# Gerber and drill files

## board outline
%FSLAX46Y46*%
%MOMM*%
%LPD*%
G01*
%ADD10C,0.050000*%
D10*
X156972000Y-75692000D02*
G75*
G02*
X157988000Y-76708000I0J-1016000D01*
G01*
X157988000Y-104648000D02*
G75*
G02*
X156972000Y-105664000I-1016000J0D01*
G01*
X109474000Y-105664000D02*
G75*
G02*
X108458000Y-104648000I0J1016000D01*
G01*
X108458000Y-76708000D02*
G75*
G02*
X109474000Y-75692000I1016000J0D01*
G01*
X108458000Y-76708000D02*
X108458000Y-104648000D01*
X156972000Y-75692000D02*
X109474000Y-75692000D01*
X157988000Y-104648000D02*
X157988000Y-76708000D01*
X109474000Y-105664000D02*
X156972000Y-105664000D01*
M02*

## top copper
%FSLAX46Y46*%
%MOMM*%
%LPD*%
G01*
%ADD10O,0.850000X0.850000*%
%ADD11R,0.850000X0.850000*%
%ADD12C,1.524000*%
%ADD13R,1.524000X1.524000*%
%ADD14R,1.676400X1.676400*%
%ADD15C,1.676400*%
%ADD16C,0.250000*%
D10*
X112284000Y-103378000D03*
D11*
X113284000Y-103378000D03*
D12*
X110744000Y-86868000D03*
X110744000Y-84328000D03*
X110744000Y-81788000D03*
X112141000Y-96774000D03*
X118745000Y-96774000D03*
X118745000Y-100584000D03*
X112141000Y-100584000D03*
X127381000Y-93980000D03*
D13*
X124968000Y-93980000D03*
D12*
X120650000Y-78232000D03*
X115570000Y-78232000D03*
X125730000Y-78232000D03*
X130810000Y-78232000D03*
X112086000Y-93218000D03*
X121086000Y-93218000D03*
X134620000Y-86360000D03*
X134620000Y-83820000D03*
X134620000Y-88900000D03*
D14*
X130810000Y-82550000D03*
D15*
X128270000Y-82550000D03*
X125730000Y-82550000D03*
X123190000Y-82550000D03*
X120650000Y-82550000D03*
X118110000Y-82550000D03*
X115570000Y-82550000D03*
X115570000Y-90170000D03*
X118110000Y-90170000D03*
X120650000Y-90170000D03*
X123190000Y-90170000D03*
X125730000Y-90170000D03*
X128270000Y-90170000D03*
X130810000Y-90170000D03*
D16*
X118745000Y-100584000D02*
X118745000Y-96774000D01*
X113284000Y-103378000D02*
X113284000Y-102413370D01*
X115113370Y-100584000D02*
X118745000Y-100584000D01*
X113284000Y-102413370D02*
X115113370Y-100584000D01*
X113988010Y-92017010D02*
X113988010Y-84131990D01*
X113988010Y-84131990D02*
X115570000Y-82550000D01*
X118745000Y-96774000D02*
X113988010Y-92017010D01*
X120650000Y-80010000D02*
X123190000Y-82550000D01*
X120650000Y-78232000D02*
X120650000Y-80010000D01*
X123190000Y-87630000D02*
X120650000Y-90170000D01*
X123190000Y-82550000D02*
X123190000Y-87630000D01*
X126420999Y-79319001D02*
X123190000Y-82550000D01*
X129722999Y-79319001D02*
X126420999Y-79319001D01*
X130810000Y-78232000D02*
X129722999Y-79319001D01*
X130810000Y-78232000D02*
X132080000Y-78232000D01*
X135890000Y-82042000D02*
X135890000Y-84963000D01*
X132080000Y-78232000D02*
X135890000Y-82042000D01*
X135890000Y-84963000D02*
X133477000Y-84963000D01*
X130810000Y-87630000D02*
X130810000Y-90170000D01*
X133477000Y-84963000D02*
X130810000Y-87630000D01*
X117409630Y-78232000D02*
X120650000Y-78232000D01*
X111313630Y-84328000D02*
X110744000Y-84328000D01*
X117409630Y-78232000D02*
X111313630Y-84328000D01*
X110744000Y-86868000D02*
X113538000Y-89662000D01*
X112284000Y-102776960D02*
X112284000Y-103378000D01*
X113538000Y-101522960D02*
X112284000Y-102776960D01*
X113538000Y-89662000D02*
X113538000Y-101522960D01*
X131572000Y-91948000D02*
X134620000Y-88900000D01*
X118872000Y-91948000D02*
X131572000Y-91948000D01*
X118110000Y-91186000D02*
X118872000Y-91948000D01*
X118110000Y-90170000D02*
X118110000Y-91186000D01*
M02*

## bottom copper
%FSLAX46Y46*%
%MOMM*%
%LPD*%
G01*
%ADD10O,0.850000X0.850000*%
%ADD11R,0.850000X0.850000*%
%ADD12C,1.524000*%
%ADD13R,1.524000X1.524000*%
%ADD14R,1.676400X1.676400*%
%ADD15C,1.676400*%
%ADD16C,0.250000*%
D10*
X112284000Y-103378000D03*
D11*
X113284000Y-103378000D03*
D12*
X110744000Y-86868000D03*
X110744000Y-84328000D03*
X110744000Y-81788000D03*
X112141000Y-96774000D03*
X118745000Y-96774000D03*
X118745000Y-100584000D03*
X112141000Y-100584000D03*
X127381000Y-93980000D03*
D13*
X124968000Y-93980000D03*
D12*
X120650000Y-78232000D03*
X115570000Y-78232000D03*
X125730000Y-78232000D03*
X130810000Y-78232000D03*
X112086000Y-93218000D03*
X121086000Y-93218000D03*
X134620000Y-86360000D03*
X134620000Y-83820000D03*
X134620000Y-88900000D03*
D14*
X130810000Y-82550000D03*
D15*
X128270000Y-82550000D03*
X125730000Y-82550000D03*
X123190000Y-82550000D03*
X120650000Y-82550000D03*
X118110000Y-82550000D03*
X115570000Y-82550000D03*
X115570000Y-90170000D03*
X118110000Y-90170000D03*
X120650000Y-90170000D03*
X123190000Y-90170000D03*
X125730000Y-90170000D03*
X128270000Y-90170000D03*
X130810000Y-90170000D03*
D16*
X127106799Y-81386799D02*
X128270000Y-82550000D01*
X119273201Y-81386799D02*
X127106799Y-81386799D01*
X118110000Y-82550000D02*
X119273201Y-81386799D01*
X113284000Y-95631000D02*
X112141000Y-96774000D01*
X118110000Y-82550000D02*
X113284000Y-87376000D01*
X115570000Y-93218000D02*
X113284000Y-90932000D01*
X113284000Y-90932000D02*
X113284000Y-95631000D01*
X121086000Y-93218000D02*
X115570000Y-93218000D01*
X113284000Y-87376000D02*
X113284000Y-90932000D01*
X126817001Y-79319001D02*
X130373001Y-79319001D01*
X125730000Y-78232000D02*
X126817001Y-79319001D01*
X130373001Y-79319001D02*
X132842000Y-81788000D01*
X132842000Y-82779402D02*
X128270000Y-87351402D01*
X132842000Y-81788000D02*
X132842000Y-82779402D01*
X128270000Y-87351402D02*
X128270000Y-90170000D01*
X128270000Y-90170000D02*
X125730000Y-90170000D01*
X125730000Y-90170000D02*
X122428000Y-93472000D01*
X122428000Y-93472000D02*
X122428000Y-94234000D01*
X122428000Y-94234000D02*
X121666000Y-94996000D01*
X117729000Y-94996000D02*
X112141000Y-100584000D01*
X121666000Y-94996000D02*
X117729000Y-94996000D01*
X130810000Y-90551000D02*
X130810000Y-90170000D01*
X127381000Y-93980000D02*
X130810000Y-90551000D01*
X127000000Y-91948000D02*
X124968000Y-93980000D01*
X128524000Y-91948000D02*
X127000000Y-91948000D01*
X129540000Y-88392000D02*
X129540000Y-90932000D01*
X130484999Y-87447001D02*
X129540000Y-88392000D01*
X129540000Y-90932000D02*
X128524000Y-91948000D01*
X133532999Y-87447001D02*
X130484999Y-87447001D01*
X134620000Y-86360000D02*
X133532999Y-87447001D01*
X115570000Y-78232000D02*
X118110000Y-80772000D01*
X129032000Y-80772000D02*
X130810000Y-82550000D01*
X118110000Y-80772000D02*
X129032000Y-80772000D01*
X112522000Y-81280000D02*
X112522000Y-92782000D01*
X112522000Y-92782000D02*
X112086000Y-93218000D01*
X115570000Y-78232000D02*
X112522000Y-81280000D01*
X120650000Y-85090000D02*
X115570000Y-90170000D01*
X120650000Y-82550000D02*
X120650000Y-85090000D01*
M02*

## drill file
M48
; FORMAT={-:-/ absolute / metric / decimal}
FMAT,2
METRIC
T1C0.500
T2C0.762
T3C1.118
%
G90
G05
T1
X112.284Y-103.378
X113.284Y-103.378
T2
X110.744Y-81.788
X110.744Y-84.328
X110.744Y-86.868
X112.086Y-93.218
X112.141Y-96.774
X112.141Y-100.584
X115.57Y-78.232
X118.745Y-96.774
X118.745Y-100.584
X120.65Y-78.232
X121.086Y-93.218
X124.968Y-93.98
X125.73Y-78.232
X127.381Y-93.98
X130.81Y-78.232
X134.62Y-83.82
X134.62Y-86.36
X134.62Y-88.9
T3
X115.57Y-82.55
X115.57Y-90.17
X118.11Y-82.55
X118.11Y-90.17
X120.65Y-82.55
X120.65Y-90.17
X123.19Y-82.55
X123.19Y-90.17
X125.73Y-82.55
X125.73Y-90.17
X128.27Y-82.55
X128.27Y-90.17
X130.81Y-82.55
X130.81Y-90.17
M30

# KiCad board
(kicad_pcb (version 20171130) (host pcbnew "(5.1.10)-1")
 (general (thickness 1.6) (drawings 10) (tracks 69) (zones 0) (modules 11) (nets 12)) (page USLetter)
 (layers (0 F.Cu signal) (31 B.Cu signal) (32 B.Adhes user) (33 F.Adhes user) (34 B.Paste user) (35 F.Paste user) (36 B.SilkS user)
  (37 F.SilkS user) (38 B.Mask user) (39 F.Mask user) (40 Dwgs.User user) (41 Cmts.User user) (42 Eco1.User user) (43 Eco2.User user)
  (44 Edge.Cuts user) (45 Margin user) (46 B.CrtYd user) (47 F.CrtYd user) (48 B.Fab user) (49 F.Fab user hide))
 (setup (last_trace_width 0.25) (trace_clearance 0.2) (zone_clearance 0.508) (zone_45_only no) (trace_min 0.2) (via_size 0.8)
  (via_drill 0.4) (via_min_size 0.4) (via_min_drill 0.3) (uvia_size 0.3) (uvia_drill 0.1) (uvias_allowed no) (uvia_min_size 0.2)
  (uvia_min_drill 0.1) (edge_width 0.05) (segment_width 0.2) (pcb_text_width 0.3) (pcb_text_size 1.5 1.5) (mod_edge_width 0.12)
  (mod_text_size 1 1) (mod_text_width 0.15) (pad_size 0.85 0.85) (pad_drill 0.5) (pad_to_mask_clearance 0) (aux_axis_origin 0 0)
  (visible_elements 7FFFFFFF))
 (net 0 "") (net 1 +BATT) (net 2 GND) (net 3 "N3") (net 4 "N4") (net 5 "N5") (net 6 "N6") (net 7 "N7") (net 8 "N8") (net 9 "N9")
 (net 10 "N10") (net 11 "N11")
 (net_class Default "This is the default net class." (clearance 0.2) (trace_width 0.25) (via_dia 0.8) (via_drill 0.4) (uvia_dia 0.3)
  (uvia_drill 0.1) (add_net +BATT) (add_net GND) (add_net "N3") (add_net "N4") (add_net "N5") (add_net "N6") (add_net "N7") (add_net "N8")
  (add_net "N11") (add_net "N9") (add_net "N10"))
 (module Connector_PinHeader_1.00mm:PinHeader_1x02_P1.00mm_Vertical (layer F.Cu) (at 113.284 103.378 270)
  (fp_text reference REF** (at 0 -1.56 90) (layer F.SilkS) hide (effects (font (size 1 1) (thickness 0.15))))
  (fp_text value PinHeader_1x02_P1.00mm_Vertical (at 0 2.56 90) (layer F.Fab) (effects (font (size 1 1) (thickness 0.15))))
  (pad 2 thru_hole oval (at 0 1 270) (size 0.85 0.85) (drill 0.5) (layers *.Cu *.Mask) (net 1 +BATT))
  (pad 1 thru_hole rect (at 0 0 270) (size 0.85 0.85) (drill 0.5) (layers *.Cu *.Mask) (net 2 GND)))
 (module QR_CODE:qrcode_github (layer F.Cu) (at 146.304 89.916)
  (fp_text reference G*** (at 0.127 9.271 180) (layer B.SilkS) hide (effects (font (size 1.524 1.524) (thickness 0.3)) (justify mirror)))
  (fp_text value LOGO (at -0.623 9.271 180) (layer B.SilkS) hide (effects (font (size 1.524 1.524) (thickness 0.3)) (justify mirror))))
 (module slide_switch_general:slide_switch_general (layer F.Cu) (at 110.744 84.328 270)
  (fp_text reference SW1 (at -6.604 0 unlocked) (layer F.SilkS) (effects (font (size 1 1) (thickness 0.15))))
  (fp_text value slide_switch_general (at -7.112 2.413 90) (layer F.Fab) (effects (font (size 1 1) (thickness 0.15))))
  (pad 3 thru_hole circle (at 2.54 0 270) (size 1.524 1.524) (drill 0.762) (layers *.Cu *.Mask) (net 1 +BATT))
  (pad 2 thru_hole circle (at 0 0 270) (size 1.524 1.524) (drill 0.762) (layers *.Cu *.Mask) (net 1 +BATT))
  (pad 1 thru_hole circle (at -2.54 0 270) (size 1.524 1.524) (drill 0.762) (layers *.Cu *.Mask)))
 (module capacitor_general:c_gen (layer F.Cu) (at 115.57 96.774)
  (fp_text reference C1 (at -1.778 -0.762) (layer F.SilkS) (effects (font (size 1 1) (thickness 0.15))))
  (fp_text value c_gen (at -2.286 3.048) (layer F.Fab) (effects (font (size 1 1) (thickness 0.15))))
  (pad 1 thru_hole circle (at -3.429 0) (size 1.524 1.524) (drill 0.762) (layers *.Cu *.Mask) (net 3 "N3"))
  (pad 2 thru_hole circle (at 3.175 0) (size 1.524 1.524) (drill 0.762) (layers *.Cu *.Mask) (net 2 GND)))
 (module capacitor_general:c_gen (layer F.Cu) (at 115.57 100.584)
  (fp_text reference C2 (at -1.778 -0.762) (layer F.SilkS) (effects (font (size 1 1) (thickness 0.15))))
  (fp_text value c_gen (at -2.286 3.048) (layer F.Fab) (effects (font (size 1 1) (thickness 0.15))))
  (pad 2 thru_hole circle (at 3.175 0) (size 1.524 1.524) (drill 0.762) (layers *.Cu *.Mask) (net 2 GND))
  (pad 1 thru_hole circle (at -3.429 0) (size 1.524 1.524) (drill 0.762) (layers *.Cu *.Mask) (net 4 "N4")))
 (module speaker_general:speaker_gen (layer F.Cu) (at 126.238 93.98 180)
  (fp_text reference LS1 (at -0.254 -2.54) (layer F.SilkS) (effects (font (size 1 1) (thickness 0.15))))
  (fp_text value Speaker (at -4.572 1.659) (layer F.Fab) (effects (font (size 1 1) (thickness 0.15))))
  (pad 1 thru_hole circle (at -1.143 0 180) (size 1.524 1.524) (drill 0.762) (layers *.Cu *.Mask) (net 1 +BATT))
  (pad 2 thru_hole rect (at 1.27 0 180) (size 1.524 1.524) (drill 0.762) (layers *.Cu *.Mask) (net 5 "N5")))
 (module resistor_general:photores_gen (layer F.Cu) (at 118.11 78.232 180)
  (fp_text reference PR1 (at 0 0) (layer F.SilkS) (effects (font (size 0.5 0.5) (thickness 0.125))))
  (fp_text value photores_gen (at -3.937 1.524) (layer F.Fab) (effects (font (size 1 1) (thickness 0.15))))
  (pad 1 thru_hole circle (at -2.54 0 180) (size 1.524 1.524) (drill 0.762) (layers *.Cu *.Mask) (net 1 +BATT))
  (pad 2 thru_hole circle (at 2.54 0 180) (size 1.524 1.524) (drill 0.762) (layers *.Cu *.Mask) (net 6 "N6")))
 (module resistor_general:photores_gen (layer F.Cu) (at 128.27 78.232 180)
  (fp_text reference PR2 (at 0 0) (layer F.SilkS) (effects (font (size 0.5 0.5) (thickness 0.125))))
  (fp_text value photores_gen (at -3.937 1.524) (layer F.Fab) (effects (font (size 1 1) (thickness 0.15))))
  (pad 2 thru_hole circle (at 2.54 0 180) (size 1.524 1.524) (drill 0.762) (layers *.Cu *.Mask) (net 4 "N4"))
  (pad 1 thru_hole circle (at -2.54 0 180) (size 1.524 1.524) (drill 0.762) (layers *.Cu *.Mask) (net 1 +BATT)))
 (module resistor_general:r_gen (layer F.Cu) (at 116.586 93.218)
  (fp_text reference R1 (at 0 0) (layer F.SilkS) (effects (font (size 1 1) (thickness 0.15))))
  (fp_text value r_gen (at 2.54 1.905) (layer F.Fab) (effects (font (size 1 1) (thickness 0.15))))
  (pad 1 thru_hole circle (at -4.5 0) (size 1.524 1.524) (drill 0.762) (layers *.Cu *.Mask) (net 6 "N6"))
  (pad 2 thru_hole circle (at 4.5 0) (size 1.524 1.524) (drill 0.762) (layers *.Cu *.Mask) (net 3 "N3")))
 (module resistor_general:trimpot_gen (layer F.Cu) (at 133.604 86.36 270)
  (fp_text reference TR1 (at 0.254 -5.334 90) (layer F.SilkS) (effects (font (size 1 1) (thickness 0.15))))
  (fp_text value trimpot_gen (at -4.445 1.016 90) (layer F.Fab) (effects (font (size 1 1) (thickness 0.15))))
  (pad 2 thru_hole circle (at 0 -1.016 270) (size 1.524 1.524) (drill 0.762) (layers *.Cu *.Mask) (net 5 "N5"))
  (pad 1 thru_hole circle (at -2.54 -1.016 270) (size 1.524 1.524) (drill 0.762) (layers *.Cu *.Mask) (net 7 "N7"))
  (pad 3 thru_hole circle (at 2.54 -1.016 270) (size 1.524 1.524) (drill 0.762) (layers *.Cu *.Mask) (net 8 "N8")))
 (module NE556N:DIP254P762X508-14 (layer F.Cu) (at 115.57 90.17 270)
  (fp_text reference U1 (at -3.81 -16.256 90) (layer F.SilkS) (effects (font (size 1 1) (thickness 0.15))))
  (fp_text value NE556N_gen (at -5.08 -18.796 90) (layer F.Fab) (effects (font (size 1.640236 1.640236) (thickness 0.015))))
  (pad 1 thru_hole rect (at -7.62 -15.24 270) (size 1.6764 1.6764) (drill 1.1176) (layers *.Cu *.Mask) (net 6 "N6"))
  (pad 2 thru_hole circle (at -7.62 -12.7 270) (size 1.6764 1.6764) (drill 1.1176) (layers *.Cu *.Mask) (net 3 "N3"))
  (pad 3 thru_hole circle (at -7.62 -10.16 270) (size 1.6764 1.6764) (drill 1.1176) (layers *.Cu *.Mask) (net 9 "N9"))
  (pad 4 thru_hole circle (at -7.62 -7.62 270) (size 1.6764 1.6764) (drill 1.1176) (layers *.Cu *.Mask) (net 1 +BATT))
  (pad 5 thru_hole circle (at -7.62 -5.08 270) (size 1.6764 1.6764) (drill 1.1176) (layers *.Cu *.Mask) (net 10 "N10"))
  (pad 6 thru_hole circle (at -7.62 -2.54 270) (size 1.6764 1.6764) (drill 1.1176) (layers *.Cu *.Mask) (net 3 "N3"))
  (pad 7 thru_hole circle (at -7.62 0 270) (size 1.6764 1.6764) (drill 1.1176) (layers *.Cu *.Mask) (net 2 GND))
  (pad 8 thru_hole circle (at 0 0 270) (size 1.6764 1.6764) (drill 1.1176) (layers *.Cu *.Mask) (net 10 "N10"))
  (pad 9 thru_hole circle (at 0 -2.54 270) (size 1.6764 1.6764) (drill 1.1176) (layers *.Cu *.Mask) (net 8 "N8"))
  (pad 10 thru_hole circle (at 0 -5.08 270) (size 1.6764 1.6764) (drill 1.1176) (layers *.Cu *.Mask) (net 1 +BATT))
  (pad 11 thru_hole circle (at 0 -7.62 270) (size 1.6764 1.6764) (drill 1.1176) (layers *.Cu *.Mask) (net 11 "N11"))
  (pad 12 thru_hole circle (at 0 -10.16 270) (size 1.6764 1.6764) (drill 1.1176) (layers *.Cu *.Mask) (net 4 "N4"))
  (pad 13 thru_hole circle (at 0 -12.7 270) (size 1.6764 1.6764) (drill 1.1176) (layers *.Cu *.Mask) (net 4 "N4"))
  (pad 14 thru_hole circle (at 0 -15.24 270) (size 1.6764 1.6764) (drill 1.1176) (layers *.Cu *.Mask) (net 1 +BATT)))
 (gr_arc (start 156.972 76.708) (end 157.988 76.708) (angle -90) (layer Edge.Cuts) (width 0.05))
 (gr_arc (start 156.972 104.648) (end 156.972 105.664) (angle -90) (layer Edge.Cuts) (width 0.05))
 (gr_arc (start 109.474 104.648) (end 108.458 104.648) (angle -90) (layer Edge.Cuts) (width 0.05))
 (gr_arc (start 109.474 76.708) (end 109.474 75.692) (angle -90) (layer Edge.Cuts) (width 0.05))
 (gr_line (start 108.458 76.708) (end 108.458 104.648) (layer Edge.Cuts) (width 0.05))
 (gr_line (start 156.972 75.692) (end 109.474 75.692) (layer Edge.Cuts) (width 0.05))
 (gr_line (start 157.988 104.648) (end 157.988 76.708) (layer Edge.Cuts) (width 0.05))
 (gr_line (start 109.474 105.664) (end 156.972 105.664) (layer Edge.Cuts) (width 0.05))
 (segment (start 127.106799 81.386799) (end 128.27 82.55) (width 0.25) (layer B.Cu) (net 3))
 (segment (start 119.273201 81.386799) (end 127.106799 81.386799) (width 0.25) (layer B.Cu) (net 3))
 (segment (start 118.11 82.55) (end 119.273201 81.386799) (width 0.25) (layer B.Cu) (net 3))
 (segment (start 113.284 95.631) (end 112.141 96.774) (width 0.25) (layer B.Cu) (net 3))
 (segment (start 118.11 82.55) (end 113.284 87.376) (width 0.25) (layer B.Cu) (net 3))
 (segment (start 115.57 93.218) (end 113.284 90.932) (width 0.25) (layer B.Cu) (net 3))
 (segment (start 113.284 90.932) (end 113.284 95.631) (width 0.25) (layer B.Cu) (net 3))
 (segment (start 121.086 93.218) (end 115.57 93.218) (width 0.25) (layer B.Cu) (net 3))
 (segment (start 113.284 87.376) (end 113.284 90.932) (width 0.25) (layer B.Cu) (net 3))
 (segment (start 118.745 100.584) (end 118.745 96.774) (width 0.25) (layer F.Cu) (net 2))
 (segment (start 113.284 103.378) (end 113.284 102.41337) (width 0.25) (layer F.Cu) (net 2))
 (segment (start 115.11337 100.584) (end 118.745 100.584) (width 0.25) (layer F.Cu) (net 2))
 (segment (start 113.284 102.41337) (end 115.11337 100.584) (width 0.25) (layer F.Cu) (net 2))
 (segment (start 113.98801 92.01701) (end 113.98801 84.13199) (width 0.25) (layer F.Cu) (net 2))
 (segment (start 113.98801 84.13199) (end 115.57 82.55) (width 0.25) (layer F.Cu) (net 2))
 (segment (start 118.745 96.774) (end 113.98801 92.01701) (width 0.25) (layer F.Cu) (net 2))
 (segment (start 126.817001 79.319001) (end 130.373001 79.319001) (width 0.25) (layer B.Cu) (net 4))
 (segment (start 125.73 78.232) (end 126.817001 79.319001) (width 0.25) (layer B.Cu) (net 4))
 (segment (start 130.373001 79.319001) (end 132.842 81.788) (width 0.25) (layer B.Cu) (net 4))
 (segment (start 132.842 82.779402) (end 128.27 87.351402) (width 0.25) (layer B.Cu) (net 4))
 (segment (start 132.842 81.788) (end 132.842 82.779402) (width 0.25) (layer B.Cu) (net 4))
 (segment (start 128.27 87.351402) (end 128.27 90.17) (width 0.25) (layer B.Cu) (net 4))
 (segment (start 128.27 90.17) (end 125.73 90.17) (width 0.25) (layer B.Cu) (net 4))
 (segment (start 125.73 90.17) (end 122.428 93.472) (width 0.25) (layer B.Cu) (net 4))
 (segment (start 122.428 93.472) (end 122.428 94.234) (width 0.25) (layer B.Cu) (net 4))
 (segment (start 122.428 94.234) (end 121.666 94.996) (width 0.25) (layer B.Cu) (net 4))
 (segment (start 117.729 94.996) (end 112.141 100.584) (width 0.25) (layer B.Cu) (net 4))
 (segment (start 121.666 94.996) (end 117.729 94.996) (width 0.25) (layer B.Cu) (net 4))
 (segment (start 120.65 80.01) (end 123.19 82.55) (width 0.25) (layer F.Cu) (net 1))
 (segment (start 120.65 78.232) (end 120.65 80.01) (width 0.25) (layer F.Cu) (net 1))
 (segment (start 123.19 87.63) (end 120.65 90.17) (width 0.25) (layer F.Cu) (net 1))
 (segment (start 123.19 82.55) (end 123.19 87.63) (width 0.25) (layer F.Cu) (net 1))
 (segment (start 126.420999 79.319001) (end 123.19 82.55) (width 0.25) (layer F.Cu) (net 1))
 (segment (start 129.722999 79.319001) (end 126.420999 79.319001) (width 0.25) (layer F.Cu) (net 1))
 (segment (start 130.81 78.232) (end 129.722999 79.319001) (width 0.25) (layer F.Cu) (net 1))
 (segment (start 130.81 78.232) (end 132.08 78.232) (width 0.25) (layer F.Cu) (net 1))
 (segment (start 135.89 82.042) (end 135.89 84.963) (width 0.25) (layer F.Cu) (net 1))
 (segment (start 132.08 78.232) (end 135.89 82.042) (width 0.25) (layer F.Cu) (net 1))
 (segment (start 135.89 84.963) (end 133.477 84.963) (width 0.25) (layer F.Cu) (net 1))
 (segment (start 130.81 87.63) (end 130.81 90.17) (width 0.25) (layer F.Cu) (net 1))
 (segment (start 133.477 84.963) (end 130.81 87.63) (width 0.25) (layer F.Cu) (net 1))
 (segment (start 130.81 90.551) (end 130.81 90.17) (width 0.25) (layer B.Cu) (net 1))
 (segment (start 127.381 93.98) (end 130.81 90.551) (width 0.25) (layer B.Cu) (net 1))
 (segment (start 117.40963 78.232) (end 120.65 78.232) (width 0.25) (layer F.Cu) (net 1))
 (segment (start 111.31363 84.328) (end 110.744 84.328) (width 0.25) (layer F.Cu) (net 1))
 (segment (start 117.40963 78.232) (end 111.31363 84.328) (width 0.25) (layer F.Cu) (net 1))
 (segment (start 110.744 86.868) (end 113.538 89.662) (width 0.25) (layer F.Cu) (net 1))
 (segment (start 112.284 102.77696) (end 112.284 103.378) (width 0.25) (layer F.Cu) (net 1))
 (segment (start 113.538 101.52296) (end 112.284 102.77696) (width 0.25) (layer F.Cu) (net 1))
 (segment (start 113.538 89.662) (end 113.538 101.52296) (width 0.25) (layer F.Cu) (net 1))
 (segment (start 127 91.948) (end 124.968 93.98) (width 0.25) (layer B.Cu) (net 5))
 (segment (start 128.524 91.948) (end 127 91.948) (width 0.25) (layer B.Cu) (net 5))
 (segment (start 129.54 88.392) (end 129.54 90.932) (width 0.25) (layer B.Cu) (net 5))
 (segment (start 130.484999 87.447001) (end 129.54 88.392) (width 0.25) (layer B.Cu) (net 5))
 (segment (start 129.54 90.932) (end 128.524 91.948) (width 0.25) (layer B.Cu) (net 5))
 (segment (start 133.532999 87.447001) (end 130.484999 87.447001) (width 0.25) (layer B.Cu) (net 5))
 (segment (start 134.62 86.36) (end 133.532999 87.447001) (width 0.25) (layer B.Cu) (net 5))
 (segment (start 115.57 78.232) (end 118.11 80.772) (width 0.25) (layer B.Cu) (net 6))
 (segment (start 129.032 80.772) (end 130.81 82.55) (width 0.25) (layer B.Cu) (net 6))
 (segment (start 118.11 80.772) (end 129.032 80.772) (width 0.25) (layer B.Cu) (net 6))
 (segment (start 112.522 81.28) (end 112.522 92.782) (width 0.25) (layer B.Cu) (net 6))
 (segment (start 112.522 92.782) (end 112.086 93.218) (width 0.25) (layer B.Cu) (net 6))
 (segment (start 115.57 78.232) (end 112.522 81.28) (width 0.25) (layer B.Cu) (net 6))
 (segment (start 131.572 91.948) (end 134.62 88.9) (width 0.25) (layer F.Cu) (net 8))
 (segment (start 118.872 91.948) (end 131.572 91.948) (width 0.25) (layer F.Cu) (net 8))
 (segment (start 118.11 91.186) (end 118.872 91.948) (width 0.25) (layer F.Cu) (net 8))
 (segment (start 118.11 90.17) (end 118.11 91.186) (width 0.25) (layer F.Cu) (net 8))
 (segment (start 120.65 85.09) (end 115.57 90.17) (width 0.25) (layer B.Cu) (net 10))
 (segment (start 120.65 82.55) (end 120.65 85.09) (width 0.25) (layer B.Cu) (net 10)))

